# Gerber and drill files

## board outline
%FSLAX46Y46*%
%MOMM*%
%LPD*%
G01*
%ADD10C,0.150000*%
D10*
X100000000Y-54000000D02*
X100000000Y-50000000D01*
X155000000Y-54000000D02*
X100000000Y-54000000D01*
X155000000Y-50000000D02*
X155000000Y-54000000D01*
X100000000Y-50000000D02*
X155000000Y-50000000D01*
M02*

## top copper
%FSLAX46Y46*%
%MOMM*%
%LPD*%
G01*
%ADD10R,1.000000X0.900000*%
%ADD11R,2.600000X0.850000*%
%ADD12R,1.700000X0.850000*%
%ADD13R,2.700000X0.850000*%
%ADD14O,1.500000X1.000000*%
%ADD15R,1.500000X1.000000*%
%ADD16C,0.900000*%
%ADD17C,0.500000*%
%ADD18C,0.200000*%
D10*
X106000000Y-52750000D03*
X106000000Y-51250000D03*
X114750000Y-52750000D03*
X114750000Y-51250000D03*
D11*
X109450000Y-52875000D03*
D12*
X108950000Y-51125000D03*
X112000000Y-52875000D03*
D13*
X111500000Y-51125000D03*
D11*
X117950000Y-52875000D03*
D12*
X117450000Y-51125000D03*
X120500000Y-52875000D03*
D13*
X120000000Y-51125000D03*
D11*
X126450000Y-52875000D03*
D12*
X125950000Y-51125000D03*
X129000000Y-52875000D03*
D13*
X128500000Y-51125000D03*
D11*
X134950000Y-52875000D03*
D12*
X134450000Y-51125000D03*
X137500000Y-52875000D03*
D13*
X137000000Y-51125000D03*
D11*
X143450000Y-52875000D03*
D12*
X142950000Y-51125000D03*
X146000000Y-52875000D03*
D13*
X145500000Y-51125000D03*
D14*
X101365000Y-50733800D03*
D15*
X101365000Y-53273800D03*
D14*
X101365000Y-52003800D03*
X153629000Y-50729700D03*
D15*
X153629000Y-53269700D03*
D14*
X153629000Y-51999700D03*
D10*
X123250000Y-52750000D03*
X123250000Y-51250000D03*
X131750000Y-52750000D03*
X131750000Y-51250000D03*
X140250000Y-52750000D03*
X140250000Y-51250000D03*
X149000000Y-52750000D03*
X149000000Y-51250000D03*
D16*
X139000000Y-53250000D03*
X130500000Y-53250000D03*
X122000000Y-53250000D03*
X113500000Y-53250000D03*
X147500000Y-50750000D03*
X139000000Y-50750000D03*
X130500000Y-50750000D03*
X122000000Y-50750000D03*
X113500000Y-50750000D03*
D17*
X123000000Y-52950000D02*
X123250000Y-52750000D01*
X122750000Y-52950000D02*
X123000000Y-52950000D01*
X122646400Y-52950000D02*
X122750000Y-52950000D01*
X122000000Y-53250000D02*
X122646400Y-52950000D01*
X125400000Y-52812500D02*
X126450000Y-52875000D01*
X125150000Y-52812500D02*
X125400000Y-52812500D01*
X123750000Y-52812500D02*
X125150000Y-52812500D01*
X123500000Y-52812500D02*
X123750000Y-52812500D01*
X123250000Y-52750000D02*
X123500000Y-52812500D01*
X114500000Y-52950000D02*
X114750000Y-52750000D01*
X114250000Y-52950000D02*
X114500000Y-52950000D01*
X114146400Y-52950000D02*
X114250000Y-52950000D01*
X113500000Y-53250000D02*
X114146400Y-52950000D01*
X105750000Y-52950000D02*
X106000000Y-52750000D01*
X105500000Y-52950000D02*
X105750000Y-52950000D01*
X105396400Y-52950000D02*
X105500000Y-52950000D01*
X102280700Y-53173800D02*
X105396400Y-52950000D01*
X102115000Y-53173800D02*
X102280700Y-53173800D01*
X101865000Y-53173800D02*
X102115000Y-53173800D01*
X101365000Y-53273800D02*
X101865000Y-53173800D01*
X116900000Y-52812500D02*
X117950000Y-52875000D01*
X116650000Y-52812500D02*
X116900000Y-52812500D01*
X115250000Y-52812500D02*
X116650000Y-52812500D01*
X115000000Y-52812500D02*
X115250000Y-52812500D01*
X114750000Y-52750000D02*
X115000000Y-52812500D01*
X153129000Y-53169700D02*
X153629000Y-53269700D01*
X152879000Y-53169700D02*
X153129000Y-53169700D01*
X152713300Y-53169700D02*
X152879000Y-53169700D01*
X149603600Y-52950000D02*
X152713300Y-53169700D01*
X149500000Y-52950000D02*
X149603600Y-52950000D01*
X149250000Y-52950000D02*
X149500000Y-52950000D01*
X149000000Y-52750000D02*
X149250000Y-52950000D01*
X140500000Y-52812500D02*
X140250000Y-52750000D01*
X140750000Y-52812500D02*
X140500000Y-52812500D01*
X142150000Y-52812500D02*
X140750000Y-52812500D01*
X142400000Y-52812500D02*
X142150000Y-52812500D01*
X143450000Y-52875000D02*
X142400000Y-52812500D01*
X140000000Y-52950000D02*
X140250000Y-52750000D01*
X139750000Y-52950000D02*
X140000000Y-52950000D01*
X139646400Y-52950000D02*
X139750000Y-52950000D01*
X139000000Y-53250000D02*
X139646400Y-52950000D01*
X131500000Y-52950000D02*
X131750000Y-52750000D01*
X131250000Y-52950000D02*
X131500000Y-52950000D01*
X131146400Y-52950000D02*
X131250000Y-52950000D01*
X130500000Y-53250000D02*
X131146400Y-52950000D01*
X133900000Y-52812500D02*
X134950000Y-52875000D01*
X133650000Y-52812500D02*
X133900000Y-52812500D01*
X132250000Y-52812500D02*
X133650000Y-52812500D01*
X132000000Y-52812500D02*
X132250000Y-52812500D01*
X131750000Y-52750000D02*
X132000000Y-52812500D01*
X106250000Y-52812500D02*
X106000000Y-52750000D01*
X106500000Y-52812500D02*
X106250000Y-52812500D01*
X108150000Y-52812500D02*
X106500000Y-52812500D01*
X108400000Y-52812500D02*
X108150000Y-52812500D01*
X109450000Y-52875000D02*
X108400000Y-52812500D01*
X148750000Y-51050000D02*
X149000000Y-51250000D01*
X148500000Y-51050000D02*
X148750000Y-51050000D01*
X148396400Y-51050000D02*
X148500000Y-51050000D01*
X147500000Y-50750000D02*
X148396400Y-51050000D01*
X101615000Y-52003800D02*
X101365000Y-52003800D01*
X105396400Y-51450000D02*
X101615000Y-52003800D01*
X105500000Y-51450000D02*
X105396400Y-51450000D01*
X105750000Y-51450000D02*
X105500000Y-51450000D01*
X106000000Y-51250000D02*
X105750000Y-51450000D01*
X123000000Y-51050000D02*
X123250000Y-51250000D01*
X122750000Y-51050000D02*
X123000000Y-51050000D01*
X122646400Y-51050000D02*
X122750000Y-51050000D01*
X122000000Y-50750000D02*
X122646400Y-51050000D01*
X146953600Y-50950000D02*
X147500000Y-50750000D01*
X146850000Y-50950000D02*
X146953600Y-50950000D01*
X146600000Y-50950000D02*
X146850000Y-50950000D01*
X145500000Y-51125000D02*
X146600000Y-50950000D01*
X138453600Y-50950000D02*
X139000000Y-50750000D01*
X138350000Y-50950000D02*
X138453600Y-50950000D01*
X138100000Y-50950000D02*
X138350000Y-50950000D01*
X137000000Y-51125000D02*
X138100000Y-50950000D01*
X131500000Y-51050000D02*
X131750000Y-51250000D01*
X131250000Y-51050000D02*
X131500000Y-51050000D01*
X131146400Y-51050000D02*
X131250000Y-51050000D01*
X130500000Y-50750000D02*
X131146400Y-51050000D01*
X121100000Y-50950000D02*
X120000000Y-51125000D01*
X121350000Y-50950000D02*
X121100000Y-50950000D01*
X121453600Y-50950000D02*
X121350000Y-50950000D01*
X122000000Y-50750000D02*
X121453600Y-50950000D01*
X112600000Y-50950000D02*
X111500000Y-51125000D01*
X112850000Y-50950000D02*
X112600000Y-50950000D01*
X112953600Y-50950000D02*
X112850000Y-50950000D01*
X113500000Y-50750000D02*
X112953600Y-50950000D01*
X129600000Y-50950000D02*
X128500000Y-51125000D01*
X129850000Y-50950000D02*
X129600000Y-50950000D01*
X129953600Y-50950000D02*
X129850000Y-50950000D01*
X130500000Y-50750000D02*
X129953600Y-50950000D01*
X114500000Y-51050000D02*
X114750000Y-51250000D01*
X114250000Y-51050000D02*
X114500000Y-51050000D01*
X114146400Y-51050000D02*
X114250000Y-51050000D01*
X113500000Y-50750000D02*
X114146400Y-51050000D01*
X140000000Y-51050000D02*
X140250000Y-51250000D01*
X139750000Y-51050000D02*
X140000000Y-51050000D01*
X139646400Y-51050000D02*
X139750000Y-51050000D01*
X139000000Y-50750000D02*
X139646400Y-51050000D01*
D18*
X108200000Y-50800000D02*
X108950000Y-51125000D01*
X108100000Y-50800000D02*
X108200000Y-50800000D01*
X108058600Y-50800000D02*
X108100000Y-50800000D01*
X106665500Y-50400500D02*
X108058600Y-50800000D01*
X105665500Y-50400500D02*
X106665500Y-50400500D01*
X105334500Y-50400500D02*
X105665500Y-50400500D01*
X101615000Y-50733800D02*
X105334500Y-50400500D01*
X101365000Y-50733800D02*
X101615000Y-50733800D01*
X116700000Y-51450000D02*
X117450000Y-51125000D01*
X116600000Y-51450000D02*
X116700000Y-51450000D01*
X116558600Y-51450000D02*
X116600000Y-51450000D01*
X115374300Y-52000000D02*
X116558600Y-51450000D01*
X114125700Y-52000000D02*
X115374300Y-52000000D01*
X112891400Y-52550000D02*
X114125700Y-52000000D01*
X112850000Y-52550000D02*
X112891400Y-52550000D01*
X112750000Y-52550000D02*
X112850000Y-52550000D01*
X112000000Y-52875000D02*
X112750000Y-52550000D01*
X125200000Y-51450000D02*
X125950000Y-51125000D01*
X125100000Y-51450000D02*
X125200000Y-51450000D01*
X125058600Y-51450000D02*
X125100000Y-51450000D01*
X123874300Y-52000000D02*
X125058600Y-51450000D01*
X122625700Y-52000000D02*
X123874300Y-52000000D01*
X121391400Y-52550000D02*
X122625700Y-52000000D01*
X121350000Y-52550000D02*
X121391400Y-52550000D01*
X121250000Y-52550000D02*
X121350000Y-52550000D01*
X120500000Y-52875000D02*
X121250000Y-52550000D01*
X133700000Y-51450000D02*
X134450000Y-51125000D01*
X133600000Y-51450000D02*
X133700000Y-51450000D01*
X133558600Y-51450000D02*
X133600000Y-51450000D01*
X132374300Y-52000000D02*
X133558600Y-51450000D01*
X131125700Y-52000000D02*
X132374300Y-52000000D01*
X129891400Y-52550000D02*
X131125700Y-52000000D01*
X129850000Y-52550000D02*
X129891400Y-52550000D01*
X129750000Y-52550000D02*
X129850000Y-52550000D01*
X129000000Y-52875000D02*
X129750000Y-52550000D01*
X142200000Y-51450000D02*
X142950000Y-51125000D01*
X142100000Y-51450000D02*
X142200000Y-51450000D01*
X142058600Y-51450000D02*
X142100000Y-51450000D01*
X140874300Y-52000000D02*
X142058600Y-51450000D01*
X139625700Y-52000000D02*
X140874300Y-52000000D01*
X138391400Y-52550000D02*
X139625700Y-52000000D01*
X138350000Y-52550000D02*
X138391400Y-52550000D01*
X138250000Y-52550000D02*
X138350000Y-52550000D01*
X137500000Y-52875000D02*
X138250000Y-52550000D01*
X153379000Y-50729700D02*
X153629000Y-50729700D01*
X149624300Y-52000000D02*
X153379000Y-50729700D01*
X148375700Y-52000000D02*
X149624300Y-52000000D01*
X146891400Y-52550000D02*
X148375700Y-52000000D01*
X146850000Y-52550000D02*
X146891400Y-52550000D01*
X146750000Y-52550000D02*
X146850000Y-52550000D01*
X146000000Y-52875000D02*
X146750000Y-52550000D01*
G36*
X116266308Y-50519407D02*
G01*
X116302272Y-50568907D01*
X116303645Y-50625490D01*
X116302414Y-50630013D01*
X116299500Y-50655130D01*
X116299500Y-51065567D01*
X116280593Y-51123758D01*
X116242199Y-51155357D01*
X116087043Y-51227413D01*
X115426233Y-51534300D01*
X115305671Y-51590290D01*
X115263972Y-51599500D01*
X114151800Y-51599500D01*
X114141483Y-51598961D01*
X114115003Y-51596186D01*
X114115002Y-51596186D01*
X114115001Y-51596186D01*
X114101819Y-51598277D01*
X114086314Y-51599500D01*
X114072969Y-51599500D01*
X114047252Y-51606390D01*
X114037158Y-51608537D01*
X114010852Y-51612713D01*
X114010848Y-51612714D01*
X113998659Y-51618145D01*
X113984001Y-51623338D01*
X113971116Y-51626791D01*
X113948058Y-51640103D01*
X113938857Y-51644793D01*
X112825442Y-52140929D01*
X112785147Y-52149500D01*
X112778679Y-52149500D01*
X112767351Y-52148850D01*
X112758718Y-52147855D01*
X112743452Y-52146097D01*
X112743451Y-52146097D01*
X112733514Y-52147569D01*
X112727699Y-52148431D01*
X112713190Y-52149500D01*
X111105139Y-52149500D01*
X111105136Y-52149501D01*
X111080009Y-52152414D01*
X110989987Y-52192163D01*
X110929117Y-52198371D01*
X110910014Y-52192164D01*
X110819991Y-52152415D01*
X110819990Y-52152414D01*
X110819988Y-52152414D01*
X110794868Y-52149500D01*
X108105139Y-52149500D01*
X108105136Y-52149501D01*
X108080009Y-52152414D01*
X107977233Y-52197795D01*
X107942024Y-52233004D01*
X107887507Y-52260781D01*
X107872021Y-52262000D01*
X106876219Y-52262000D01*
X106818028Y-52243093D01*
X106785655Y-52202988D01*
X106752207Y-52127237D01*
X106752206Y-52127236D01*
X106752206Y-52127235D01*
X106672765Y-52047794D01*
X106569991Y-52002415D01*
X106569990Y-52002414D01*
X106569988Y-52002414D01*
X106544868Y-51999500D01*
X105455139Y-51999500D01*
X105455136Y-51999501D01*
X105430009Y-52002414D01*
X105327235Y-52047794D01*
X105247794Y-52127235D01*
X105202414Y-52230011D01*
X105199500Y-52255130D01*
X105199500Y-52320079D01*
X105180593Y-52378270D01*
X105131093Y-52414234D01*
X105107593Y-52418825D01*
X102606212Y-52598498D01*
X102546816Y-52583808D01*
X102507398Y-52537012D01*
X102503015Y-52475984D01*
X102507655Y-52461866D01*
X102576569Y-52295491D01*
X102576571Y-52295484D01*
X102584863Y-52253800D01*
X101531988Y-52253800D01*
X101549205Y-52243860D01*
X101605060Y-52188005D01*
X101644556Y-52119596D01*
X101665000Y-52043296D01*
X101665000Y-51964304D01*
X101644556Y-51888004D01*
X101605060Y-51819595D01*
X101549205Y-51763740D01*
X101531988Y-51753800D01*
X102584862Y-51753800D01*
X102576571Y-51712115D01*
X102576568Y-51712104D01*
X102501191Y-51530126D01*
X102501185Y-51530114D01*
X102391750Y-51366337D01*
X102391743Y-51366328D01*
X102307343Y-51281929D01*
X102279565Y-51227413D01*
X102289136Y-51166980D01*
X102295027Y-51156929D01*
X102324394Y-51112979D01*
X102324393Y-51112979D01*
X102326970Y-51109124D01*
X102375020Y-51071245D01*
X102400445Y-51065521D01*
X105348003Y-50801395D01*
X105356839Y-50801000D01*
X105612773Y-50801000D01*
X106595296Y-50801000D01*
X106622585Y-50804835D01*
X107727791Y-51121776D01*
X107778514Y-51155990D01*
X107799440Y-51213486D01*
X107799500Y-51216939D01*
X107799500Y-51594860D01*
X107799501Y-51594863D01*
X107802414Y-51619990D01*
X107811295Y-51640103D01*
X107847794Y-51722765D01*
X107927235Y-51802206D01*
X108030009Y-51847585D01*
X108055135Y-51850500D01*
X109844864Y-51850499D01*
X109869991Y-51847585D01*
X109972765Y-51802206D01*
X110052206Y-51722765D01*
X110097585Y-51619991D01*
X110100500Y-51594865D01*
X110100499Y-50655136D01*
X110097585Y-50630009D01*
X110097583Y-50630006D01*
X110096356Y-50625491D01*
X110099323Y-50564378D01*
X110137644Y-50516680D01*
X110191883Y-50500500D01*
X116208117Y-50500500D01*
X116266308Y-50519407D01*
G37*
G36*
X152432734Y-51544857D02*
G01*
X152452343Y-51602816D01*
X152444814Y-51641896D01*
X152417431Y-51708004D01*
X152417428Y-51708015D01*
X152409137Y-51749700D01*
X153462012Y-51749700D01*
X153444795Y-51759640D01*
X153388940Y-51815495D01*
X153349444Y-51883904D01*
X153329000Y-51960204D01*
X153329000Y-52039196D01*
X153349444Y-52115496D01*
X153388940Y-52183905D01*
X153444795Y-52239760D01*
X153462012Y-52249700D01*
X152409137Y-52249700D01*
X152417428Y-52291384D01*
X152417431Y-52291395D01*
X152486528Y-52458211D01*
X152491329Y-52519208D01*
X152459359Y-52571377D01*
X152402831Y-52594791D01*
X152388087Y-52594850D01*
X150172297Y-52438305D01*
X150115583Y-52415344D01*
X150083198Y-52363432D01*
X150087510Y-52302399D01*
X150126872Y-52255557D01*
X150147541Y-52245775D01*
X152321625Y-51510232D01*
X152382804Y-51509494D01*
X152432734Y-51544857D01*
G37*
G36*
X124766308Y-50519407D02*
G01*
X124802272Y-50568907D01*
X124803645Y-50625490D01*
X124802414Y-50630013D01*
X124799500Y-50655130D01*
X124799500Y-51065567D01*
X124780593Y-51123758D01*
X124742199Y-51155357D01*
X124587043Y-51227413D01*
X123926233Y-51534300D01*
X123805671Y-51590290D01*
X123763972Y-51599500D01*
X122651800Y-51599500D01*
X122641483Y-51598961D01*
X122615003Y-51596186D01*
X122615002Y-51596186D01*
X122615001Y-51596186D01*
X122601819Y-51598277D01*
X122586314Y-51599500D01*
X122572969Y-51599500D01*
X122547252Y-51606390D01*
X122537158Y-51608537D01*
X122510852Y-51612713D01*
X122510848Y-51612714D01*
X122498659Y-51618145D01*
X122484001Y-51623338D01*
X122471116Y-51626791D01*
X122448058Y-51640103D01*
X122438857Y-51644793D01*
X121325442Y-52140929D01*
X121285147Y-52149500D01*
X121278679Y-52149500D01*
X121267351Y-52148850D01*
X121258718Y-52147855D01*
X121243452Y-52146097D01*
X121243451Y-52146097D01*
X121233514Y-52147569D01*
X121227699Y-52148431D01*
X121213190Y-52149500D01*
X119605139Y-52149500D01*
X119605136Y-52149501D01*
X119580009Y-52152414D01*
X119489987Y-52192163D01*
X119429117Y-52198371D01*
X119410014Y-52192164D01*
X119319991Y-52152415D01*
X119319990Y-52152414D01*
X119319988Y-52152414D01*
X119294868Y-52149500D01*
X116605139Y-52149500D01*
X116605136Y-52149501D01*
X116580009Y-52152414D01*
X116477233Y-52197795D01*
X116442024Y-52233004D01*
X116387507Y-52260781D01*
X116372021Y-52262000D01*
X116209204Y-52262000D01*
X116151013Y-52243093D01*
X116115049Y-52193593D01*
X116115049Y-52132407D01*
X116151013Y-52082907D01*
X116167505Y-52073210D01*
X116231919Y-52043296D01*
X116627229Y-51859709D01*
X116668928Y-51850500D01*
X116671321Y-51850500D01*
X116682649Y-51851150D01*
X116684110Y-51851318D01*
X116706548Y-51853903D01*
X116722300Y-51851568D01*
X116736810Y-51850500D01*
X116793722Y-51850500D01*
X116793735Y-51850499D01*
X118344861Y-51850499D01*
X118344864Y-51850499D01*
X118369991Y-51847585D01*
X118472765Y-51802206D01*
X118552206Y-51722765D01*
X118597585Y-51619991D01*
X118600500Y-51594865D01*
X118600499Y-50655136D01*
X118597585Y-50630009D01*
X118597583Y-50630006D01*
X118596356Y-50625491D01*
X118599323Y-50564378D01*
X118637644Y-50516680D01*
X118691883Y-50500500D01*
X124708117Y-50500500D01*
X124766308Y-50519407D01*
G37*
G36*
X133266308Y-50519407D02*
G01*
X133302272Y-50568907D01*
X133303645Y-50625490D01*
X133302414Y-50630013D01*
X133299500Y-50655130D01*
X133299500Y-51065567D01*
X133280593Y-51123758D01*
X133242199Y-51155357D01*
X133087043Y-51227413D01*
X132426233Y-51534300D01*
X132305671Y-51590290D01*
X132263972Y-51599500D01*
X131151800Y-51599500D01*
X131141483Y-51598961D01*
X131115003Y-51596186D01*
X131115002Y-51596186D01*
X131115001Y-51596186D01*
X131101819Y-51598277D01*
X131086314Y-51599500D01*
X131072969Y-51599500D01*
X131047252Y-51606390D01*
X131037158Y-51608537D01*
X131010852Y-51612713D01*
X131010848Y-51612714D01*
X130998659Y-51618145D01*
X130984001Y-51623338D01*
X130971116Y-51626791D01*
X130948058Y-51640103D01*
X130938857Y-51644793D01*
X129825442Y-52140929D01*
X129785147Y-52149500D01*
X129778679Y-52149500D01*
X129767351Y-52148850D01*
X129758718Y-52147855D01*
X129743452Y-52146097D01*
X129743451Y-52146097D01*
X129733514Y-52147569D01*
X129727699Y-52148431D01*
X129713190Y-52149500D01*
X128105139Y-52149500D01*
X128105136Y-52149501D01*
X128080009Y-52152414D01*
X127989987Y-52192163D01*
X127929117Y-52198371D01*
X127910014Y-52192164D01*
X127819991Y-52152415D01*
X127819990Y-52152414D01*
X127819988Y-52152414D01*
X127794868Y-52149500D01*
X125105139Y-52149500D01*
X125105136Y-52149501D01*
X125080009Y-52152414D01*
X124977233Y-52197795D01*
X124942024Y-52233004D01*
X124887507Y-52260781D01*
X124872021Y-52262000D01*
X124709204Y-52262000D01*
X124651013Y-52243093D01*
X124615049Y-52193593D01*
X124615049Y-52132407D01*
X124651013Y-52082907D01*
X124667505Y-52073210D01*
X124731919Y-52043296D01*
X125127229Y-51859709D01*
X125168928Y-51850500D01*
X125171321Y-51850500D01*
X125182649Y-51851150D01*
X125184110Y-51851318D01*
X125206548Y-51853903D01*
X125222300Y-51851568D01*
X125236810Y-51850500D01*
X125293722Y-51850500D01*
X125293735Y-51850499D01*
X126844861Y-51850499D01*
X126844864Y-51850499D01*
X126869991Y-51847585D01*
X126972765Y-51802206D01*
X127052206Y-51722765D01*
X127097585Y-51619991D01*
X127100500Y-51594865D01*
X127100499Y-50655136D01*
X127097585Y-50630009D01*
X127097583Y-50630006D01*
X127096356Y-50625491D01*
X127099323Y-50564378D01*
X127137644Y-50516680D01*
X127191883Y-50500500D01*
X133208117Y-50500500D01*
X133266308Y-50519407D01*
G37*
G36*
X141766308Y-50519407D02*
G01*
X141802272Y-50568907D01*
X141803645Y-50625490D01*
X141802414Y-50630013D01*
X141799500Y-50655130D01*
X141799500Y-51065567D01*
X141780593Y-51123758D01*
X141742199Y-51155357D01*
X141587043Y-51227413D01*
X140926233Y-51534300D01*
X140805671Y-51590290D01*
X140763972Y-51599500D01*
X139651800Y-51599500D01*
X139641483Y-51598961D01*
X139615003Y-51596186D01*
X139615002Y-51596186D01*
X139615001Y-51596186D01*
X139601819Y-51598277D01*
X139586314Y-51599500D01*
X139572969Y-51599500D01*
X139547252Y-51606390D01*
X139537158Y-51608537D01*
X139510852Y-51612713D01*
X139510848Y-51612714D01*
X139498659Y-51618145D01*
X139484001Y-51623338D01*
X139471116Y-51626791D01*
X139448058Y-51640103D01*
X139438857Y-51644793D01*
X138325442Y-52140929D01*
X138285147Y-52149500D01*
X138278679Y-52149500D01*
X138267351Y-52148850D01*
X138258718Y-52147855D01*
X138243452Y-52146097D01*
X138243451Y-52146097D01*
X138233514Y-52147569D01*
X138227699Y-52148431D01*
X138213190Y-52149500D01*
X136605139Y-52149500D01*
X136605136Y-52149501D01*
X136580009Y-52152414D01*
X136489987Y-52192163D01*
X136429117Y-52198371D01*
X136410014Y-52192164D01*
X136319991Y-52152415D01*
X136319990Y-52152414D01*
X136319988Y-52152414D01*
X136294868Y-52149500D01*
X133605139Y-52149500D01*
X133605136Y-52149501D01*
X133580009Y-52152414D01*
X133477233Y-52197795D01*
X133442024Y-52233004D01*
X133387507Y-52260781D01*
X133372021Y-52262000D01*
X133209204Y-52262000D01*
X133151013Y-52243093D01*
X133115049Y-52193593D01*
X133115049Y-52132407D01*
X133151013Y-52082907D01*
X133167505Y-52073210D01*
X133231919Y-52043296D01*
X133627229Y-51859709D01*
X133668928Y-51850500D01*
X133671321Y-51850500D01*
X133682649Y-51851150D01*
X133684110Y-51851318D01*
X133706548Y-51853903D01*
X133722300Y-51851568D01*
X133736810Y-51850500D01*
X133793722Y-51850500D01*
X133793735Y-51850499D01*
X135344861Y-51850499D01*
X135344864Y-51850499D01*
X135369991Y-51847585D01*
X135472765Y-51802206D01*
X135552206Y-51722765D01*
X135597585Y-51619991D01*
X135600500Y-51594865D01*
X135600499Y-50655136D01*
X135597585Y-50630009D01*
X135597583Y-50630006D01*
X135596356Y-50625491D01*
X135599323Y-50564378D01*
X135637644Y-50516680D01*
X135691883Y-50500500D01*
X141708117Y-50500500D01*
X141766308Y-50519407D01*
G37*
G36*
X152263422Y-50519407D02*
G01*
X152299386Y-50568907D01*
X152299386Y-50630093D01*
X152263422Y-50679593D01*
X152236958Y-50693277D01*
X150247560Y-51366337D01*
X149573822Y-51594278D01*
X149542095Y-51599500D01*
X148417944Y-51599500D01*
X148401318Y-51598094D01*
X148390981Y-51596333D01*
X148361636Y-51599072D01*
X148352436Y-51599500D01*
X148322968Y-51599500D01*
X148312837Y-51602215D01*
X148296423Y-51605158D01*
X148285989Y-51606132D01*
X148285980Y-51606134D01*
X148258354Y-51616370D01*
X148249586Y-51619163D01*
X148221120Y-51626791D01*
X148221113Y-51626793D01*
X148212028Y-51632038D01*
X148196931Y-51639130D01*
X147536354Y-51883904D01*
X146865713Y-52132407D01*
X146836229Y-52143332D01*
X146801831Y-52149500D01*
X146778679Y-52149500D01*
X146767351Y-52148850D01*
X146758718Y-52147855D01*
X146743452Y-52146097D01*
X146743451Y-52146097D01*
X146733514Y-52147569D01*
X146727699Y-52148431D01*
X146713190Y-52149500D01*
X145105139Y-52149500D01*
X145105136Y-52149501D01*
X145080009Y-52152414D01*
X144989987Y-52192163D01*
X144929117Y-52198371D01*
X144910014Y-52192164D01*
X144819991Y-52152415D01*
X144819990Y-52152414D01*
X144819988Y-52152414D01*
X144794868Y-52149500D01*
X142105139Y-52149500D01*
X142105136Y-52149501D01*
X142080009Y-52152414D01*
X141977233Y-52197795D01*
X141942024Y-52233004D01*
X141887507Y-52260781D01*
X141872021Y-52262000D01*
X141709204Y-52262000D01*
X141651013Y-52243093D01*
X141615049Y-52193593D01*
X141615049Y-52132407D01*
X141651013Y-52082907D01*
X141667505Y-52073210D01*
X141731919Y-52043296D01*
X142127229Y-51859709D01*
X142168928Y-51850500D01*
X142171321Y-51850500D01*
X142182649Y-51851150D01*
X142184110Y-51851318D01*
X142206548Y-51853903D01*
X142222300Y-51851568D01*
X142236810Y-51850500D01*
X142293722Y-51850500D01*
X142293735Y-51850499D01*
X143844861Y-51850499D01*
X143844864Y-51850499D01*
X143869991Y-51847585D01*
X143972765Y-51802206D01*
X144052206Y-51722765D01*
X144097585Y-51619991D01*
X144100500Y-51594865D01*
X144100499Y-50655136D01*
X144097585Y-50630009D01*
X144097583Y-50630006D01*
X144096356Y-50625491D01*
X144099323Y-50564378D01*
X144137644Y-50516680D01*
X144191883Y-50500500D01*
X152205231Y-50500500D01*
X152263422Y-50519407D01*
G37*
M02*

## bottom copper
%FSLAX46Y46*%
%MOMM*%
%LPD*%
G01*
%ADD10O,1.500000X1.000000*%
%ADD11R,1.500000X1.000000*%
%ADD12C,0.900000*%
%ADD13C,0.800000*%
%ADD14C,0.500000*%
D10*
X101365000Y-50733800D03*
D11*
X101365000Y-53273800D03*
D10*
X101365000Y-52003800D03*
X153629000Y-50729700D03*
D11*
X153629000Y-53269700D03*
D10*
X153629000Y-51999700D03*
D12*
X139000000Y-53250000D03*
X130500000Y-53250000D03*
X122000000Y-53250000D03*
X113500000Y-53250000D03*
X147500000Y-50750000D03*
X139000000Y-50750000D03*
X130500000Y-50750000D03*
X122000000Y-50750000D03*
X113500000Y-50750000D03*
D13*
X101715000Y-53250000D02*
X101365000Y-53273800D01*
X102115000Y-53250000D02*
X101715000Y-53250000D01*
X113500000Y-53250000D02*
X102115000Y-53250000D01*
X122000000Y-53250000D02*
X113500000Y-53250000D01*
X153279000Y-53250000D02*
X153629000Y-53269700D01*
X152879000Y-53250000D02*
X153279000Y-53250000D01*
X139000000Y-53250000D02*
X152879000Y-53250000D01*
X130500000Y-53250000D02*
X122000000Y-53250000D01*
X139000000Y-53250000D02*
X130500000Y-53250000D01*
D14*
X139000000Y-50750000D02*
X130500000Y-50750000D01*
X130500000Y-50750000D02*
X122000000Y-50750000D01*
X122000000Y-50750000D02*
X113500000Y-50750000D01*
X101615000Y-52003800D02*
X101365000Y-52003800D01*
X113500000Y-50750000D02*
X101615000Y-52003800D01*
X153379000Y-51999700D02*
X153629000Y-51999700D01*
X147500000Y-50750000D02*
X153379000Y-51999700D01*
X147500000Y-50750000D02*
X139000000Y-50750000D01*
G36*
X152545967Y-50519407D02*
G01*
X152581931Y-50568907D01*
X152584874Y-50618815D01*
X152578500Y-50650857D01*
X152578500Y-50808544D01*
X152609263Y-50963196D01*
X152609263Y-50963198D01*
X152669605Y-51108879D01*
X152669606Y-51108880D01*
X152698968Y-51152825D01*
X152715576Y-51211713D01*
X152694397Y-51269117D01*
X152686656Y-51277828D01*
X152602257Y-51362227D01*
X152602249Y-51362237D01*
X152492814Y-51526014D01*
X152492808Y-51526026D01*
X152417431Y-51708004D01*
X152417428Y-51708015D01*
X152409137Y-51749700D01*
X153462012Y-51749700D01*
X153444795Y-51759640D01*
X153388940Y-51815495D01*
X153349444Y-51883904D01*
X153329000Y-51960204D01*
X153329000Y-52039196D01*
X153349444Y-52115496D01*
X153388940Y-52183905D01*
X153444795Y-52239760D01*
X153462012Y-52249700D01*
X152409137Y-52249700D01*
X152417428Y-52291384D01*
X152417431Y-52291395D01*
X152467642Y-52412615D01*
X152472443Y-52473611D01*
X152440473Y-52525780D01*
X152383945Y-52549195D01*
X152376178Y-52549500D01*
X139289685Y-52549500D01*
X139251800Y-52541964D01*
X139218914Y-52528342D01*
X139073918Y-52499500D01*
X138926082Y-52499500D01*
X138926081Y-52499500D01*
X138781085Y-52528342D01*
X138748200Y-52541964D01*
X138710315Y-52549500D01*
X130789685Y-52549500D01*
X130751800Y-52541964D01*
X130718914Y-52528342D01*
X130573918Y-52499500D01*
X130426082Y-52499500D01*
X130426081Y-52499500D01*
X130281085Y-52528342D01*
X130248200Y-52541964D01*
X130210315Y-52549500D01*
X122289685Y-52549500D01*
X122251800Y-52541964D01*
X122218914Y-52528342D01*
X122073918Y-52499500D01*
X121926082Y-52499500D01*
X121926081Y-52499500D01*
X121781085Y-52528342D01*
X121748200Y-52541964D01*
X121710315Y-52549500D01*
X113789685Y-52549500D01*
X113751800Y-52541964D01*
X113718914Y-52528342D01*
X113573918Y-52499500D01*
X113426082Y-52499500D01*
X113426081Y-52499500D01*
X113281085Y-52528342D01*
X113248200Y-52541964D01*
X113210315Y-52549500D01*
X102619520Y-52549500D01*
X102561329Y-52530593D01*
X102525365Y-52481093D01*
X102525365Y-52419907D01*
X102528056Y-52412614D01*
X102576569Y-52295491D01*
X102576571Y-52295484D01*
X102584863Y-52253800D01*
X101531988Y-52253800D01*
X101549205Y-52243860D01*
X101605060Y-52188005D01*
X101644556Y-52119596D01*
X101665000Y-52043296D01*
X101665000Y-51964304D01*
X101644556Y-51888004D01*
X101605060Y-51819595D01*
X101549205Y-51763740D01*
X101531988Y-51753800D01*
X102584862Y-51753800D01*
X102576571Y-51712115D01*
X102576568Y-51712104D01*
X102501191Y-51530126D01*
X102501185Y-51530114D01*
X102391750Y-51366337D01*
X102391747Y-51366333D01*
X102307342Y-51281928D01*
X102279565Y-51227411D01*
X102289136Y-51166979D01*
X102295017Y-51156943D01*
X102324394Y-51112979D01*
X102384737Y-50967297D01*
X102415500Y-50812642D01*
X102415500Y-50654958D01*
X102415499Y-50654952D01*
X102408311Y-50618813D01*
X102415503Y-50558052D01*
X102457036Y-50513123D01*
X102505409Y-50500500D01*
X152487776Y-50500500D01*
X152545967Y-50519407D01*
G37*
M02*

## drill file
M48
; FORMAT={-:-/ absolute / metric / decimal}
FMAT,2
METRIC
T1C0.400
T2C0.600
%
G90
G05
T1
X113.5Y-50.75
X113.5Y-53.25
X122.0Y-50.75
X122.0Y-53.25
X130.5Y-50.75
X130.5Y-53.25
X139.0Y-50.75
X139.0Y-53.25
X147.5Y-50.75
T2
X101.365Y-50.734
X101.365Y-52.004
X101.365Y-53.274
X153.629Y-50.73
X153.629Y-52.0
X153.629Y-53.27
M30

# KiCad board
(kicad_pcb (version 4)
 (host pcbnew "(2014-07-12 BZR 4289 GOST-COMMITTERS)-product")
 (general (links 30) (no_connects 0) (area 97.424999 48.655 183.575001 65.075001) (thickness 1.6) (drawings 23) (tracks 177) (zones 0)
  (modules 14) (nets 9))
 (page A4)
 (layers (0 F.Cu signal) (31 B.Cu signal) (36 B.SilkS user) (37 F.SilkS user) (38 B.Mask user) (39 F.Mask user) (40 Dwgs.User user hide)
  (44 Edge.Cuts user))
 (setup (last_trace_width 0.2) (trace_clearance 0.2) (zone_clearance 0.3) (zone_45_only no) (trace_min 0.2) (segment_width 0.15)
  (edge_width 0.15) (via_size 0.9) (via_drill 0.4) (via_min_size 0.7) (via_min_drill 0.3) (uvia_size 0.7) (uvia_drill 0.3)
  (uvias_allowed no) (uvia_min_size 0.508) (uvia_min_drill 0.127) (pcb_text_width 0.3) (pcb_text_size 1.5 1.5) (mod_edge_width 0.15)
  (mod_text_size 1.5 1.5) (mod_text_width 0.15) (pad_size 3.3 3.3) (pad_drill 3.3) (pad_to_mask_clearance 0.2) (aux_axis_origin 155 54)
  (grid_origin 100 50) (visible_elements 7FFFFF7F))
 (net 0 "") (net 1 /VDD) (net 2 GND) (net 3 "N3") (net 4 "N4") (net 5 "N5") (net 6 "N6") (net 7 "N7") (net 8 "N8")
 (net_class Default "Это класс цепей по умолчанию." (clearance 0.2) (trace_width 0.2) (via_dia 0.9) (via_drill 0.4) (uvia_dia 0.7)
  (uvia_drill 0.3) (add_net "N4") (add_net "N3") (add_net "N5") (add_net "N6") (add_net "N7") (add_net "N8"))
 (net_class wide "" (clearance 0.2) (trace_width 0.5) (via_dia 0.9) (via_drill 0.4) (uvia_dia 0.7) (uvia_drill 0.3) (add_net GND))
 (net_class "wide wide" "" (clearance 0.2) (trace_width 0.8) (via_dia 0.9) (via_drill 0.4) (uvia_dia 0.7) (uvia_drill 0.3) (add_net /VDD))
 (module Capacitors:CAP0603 (layer F.Cu) (at 106 52 90)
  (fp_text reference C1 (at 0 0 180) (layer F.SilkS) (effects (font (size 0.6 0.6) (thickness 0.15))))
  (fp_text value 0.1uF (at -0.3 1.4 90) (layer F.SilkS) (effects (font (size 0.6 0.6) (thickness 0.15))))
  (pad 1 smd rect (at -0.75 0 90) (size 0.9 1) (layers F.Cu F.Mask) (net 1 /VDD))
  (pad 2 smd rect (at 0.75 0 90) (size 0.9 1) (layers F.Cu F.Mask) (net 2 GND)))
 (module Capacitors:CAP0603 (layer F.Cu) (at 114.75 52 90)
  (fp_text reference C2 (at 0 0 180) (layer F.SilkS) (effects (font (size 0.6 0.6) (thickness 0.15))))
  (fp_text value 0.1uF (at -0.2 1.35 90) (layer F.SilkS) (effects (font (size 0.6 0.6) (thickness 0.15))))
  (pad 1 smd rect (at -0.75 0 90) (size 0.9 1) (layers F.Cu F.Mask) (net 1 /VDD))
  (pad 2 smd rect (at 0.75 0 90) (size 0.9 1) (layers F.Cu F.Mask) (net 2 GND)))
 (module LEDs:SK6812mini (layer F.Cu) (at 110.5 52 180)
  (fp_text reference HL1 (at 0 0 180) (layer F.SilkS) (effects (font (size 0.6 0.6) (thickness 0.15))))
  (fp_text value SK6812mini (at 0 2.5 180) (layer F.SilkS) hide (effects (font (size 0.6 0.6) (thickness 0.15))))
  (pad 4 smd rect (at 1.05 -0.875 180) (size 2.6 0.85) (layers F.Cu F.Mask) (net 1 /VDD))
  (pad 3 smd rect (at 1.55 0.875 180) (size 1.7 0.85) (layers F.Cu F.Mask) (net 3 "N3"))
  (pad 1 smd rect (at -1.5 -0.875 180) (size 1.7 0.85) (layers F.Cu F.Mask) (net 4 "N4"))
  (pad 2 smd rect (at -1 0.875 180) (size 2.7 0.85) (layers F.Cu F.Mask) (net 2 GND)))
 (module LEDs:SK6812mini (layer F.Cu) (at 119 52 180)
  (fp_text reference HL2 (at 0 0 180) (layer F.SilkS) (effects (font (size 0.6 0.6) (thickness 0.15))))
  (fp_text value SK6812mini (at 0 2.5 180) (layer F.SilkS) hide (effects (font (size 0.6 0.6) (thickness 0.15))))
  (pad 4 smd rect (at 1.05 -0.875 180) (size 2.6 0.85) (layers F.Cu F.Mask) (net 1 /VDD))
  (pad 3 smd rect (at 1.55 0.875 180) (size 1.7 0.85) (layers F.Cu F.Mask) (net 4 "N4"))
  (pad 1 smd rect (at -1.5 -0.875 180) (size 1.7 0.85) (layers F.Cu F.Mask) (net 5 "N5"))
  (pad 2 smd rect (at -1 0.875 180) (size 2.7 0.85) (layers F.Cu F.Mask) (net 2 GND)))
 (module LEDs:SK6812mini (layer F.Cu) (at 127.5 52 180)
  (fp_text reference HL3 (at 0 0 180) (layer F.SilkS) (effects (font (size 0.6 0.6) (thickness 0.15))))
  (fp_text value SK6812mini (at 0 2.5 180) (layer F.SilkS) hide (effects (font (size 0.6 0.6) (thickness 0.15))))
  (pad 4 smd rect (at 1.05 -0.875 180) (size 2.6 0.85) (layers F.Cu F.Mask) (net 1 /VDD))
  (pad 3 smd rect (at 1.55 0.875 180) (size 1.7 0.85) (layers F.Cu F.Mask) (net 5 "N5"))
  (pad 1 smd rect (at -1.5 -0.875 180) (size 1.7 0.85) (layers F.Cu F.Mask) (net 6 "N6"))
  (pad 2 smd rect (at -1 0.875 180) (size 2.7 0.85) (layers F.Cu F.Mask) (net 2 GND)))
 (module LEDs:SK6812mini (layer F.Cu) (at 136 52 180)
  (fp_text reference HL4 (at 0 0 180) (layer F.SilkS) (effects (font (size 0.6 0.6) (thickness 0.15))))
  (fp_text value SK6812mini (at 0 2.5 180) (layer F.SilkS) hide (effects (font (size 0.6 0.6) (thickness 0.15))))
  (pad 4 smd rect (at 1.05 -0.875 180) (size 2.6 0.85) (layers F.Cu F.Mask) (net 1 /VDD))
  (pad 3 smd rect (at 1.55 0.875 180) (size 1.7 0.85) (layers F.Cu F.Mask) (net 6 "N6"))
  (pad 1 smd rect (at -1.5 -0.875 180) (size 1.7 0.85) (layers F.Cu F.Mask) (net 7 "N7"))
  (pad 2 smd rect (at -1 0.875 180) (size 2.7 0.85) (layers F.Cu F.Mask) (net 2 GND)))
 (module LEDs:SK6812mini (layer F.Cu) (at 144.5 52 180)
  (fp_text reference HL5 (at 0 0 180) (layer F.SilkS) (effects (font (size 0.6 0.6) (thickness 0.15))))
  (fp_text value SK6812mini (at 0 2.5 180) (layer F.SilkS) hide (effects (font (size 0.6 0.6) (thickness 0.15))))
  (pad 4 smd rect (at 1.05 -0.875 180) (size 2.6 0.85) (layers F.Cu F.Mask) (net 1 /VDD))
  (pad 3 smd rect (at 1.55 0.875 180) (size 1.7 0.85) (layers F.Cu F.Mask) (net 7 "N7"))
  (pad 1 smd rect (at -1.5 -0.875 180) (size 1.7 0.85) (layers F.Cu F.Mask) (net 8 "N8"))
  (pad 2 smd rect (at -1 0.875 180) (size 2.7 0.85) (layers F.Cu F.Mask) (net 2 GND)))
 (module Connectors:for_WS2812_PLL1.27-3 (layer F.Cu) (at 101.365 53.2738 90)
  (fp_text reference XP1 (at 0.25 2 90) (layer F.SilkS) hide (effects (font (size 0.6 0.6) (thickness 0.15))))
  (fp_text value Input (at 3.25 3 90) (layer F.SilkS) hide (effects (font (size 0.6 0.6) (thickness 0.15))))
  (pad 3 thru_hole oval (at 2.54 0 90) (size 1 1.5) (drill 0.6) (layers *.Cu *.Mask) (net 3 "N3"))
  (pad 1 thru_hole rect (at 0 0 90) (size 1 1.5) (drill 0.6) (layers *.Cu *.Mask) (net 1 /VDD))
  (pad 2 thru_hole oval (at 1.27 0 90) (size 1 1.5) (drill 0.6) (layers *.Cu *.Mask) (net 2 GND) (zone_connect 1)))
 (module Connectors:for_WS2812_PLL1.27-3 (layer F.Cu) (at 153.629 53.2697 90)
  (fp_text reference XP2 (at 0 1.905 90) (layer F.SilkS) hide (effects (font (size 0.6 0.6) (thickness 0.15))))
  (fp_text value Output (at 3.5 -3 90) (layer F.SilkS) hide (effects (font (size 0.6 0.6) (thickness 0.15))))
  (pad 3 thru_hole oval (at 2.54 0 90) (size 1 1.5) (drill 0.6) (layers *.Cu *.Mask) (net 8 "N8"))
  (pad 1 thru_hole rect (at 0 0 90) (size 1 1.5) (drill 0.6) (layers *.Cu *.Mask) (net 1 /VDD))
  (pad 2 thru_hole oval (at 1.27 0 90) (size 1 1.5) (drill 0.6) (layers *.Cu *.Mask) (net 2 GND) (zone_connect 1)))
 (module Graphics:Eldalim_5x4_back (layer B.Cu) (at 117.5 52)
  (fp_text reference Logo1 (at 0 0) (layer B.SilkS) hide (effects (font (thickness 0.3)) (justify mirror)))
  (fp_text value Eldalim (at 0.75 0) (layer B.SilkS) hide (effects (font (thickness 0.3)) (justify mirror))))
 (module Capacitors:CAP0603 (layer F.Cu) (at 123.25 52 90)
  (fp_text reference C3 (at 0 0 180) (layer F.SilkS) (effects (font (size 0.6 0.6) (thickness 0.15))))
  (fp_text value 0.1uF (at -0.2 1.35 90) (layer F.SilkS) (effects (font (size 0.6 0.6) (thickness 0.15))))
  (pad 1 smd rect (at -0.75 0 90) (size 0.9 1) (layers F.Cu F.Mask) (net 1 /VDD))
  (pad 2 smd rect (at 0.75 0 90) (size 0.9 1) (layers F.Cu F.Mask) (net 2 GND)))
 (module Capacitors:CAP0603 (layer F.Cu) (at 131.75 52 90)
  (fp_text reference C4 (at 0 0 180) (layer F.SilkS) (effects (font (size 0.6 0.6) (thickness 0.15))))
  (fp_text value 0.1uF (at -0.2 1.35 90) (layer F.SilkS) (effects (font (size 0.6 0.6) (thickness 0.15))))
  (pad 1 smd rect (at -0.75 0 90) (size 0.9 1) (layers F.Cu F.Mask) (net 1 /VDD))
  (pad 2 smd rect (at 0.75 0 90) (size 0.9 1) (layers F.Cu F.Mask) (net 2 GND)))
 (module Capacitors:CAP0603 (layer F.Cu) (at 140.25 52 90)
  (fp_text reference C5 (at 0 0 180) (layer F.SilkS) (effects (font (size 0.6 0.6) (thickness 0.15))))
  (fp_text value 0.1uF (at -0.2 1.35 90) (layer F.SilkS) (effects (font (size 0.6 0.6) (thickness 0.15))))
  (pad 1 smd rect (at -0.75 0 90) (size 0.9 1) (layers F.Cu F.Mask) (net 1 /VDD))
  (pad 2 smd rect (at 0.75 0 90) (size 0.9 1) (layers F.Cu F.Mask) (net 2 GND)))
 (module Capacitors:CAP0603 (layer F.Cu) (at 149 52 90)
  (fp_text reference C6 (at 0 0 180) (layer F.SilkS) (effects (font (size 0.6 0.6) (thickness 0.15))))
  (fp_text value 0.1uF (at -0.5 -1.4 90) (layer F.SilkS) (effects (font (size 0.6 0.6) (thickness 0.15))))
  (pad 1 smd rect (at -0.75 0 90) (size 0.9 1) (layers F.Cu F.Mask) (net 1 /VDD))
  (pad 2 smd rect (at 0.75 0 90) (size 0.9 1) (layers F.Cu F.Mask) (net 2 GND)))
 (gr_line (start 100 54) (end 100 50) (angle 90) (layer Edge.Cuts) (width 0.15))
 (gr_line (start 155 54) (end 100 54) (angle 90) (layer Edge.Cuts) (width 0.15))
 (gr_line (start 155 50) (end 155 54) (angle 90) (layer Edge.Cuts) (width 0.15))
 (gr_line (start 100 50) (end 155 50) (angle 90) (layer Edge.Cuts) (width 0.15)) (via (at 139 53.25) (size 0.9) (layers F.Cu B.Cu) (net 1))
 (via (at 130.5 53.25) (size 0.9) (layers F.Cu B.Cu) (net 1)) (via (at 122 53.25) (size 0.9) (layers F.Cu B.Cu) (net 1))
 (via (at 113.5 53.25) (size 0.9) (layers F.Cu B.Cu) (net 1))
 (segment (start 101.715 53.25) (end 101.365 53.2738) (width 0.8) (layer B.Cu) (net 1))
 (segment (start 102.115 53.25) (end 101.715 53.25) (width 0.8) (layer B.Cu) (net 1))
 (segment (start 113.5 53.25) (end 102.115 53.25) (width 0.8) (layer B.Cu) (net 1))
 (segment (start 122 53.25) (end 113.5 53.25) (width 0.8) (layer B.Cu) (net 1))
 (segment (start 153.279 53.25) (end 153.629 53.2697) (width 0.8) (layer B.Cu) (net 1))
 (segment (start 152.879 53.25) (end 153.279 53.25) (width 0.8) (layer B.Cu) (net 1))
 (segment (start 139 53.25) (end 152.879 53.25) (width 0.8) (layer B.Cu) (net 1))
 (segment (start 130.5 53.25) (end 122 53.25) (width 0.8) (layer B.Cu) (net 1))
 (segment (start 139 53.25) (end 130.5 53.25) (width 0.8) (layer B.Cu) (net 1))
 (segment (start 123 52.95) (end 123.25 52.75) (width 0.5) (layer F.Cu) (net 1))
 (segment (start 122.75 52.95) (end 123 52.95) (width 0.5) (layer F.Cu) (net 1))
 (segment (start 122.6464 52.95) (end 122.75 52.95) (width 0.5) (layer F.Cu) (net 1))
 (segment (start 122 53.25) (end 122.6464 52.95) (width 0.5) (layer F.Cu) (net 1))
 (segment (start 125.4 52.8125) (end 126.45 52.875) (width 0.5) (layer F.Cu) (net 1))
 (segment (start 125.15 52.8125) (end 125.4 52.8125) (width 0.5) (layer F.Cu) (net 1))
 (segment (start 123.75 52.8125) (end 125.15 52.8125) (width 0.5) (layer F.Cu) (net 1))
 (segment (start 123.5 52.8125) (end 123.75 52.8125) (width 0.5) (layer F.Cu) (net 1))
 (segment (start 123.25 52.75) (end 123.5 52.8125) (width 0.5) (layer F.Cu) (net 1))
 (segment (start 114.5 52.95) (end 114.75 52.75) (width 0.5) (layer F.Cu) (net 1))
 (segment (start 114.25 52.95) (end 114.5 52.95) (width 0.5) (layer F.Cu) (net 1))
 (segment (start 114.1464 52.95) (end 114.25 52.95) (width 0.5) (layer F.Cu) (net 1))
 (segment (start 113.5 53.25) (end 114.1464 52.95) (width 0.5) (layer F.Cu) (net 1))
 (segment (start 105.75 52.95) (end 106 52.75) (width 0.5) (layer F.Cu) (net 1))
 (segment (start 105.5 52.95) (end 105.75 52.95) (width 0.5) (layer F.Cu) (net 1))
 (segment (start 105.3964 52.95) (end 105.5 52.95) (width 0.5) (layer F.Cu) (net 1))
 (segment (start 102.2807 53.1738) (end 105.3964 52.95) (width 0.5) (layer F.Cu) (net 1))
 (segment (start 102.115 53.1738) (end 102.2807 53.1738) (width 0.5) (layer F.Cu) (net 1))
 (segment (start 101.865 53.1738) (end 102.115 53.1738) (width 0.5) (layer F.Cu) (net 1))
 (segment (start 101.365 53.2738) (end 101.865 53.1738) (width 0.5) (layer F.Cu) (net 1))
 (segment (start 116.9 52.8125) (end 117.95 52.875) (width 0.5) (layer F.Cu) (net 1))
 (segment (start 116.65 52.8125) (end 116.9 52.8125) (width 0.5) (layer F.Cu) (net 1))
 (segment (start 115.25 52.8125) (end 116.65 52.8125) (width 0.5) (layer F.Cu) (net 1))
 (segment (start 115 52.8125) (end 115.25 52.8125) (width 0.5) (layer F.Cu) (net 1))
 (segment (start 114.75 52.75) (end 115 52.8125) (width 0.5) (layer F.Cu) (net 1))
 (segment (start 153.129 53.1697) (end 153.629 53.2697) (width 0.5) (layer F.Cu) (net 1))
 (segment (start 152.879 53.1697) (end 153.129 53.1697) (width 0.5) (layer F.Cu) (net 1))
 (segment (start 152.7133 53.1697) (end 152.879 53.1697) (width 0.5) (layer F.Cu) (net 1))
 (segment (start 149.6036 52.95) (end 152.7133 53.1697) (width 0.5) (layer F.Cu) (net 1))
 (segment (start 149.5 52.95) (end 149.6036 52.95) (width 0.5) (layer F.Cu) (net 1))
 (segment (start 149.25 52.95) (end 149.5 52.95) (width 0.5) (layer F.Cu) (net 1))
 (segment (start 149 52.75) (end 149.25 52.95) (width 0.5) (layer F.Cu) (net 1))
 (segment (start 140.5 52.8125) (end 140.25 52.75) (width 0.5) (layer F.Cu) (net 1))
 (segment (start 140.75 52.8125) (end 140.5 52.8125) (width 0.5) (layer F.Cu) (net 1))
 (segment (start 142.15 52.8125) (end 140.75 52.8125) (width 0.5) (layer F.Cu) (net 1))
 (segment (start 142.4 52.8125) (end 142.15 52.8125) (width 0.5) (layer F.Cu) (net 1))
 (segment (start 143.45 52.875) (end 142.4 52.8125) (width 0.5) (layer F.Cu) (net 1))
 (segment (start 140 52.95) (end 140.25 52.75) (width 0.5) (layer F.Cu) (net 1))
 (segment (start 139.75 52.95) (end 140 52.95) (width 0.5) (layer F.Cu) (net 1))
 (segment (start 139.6464 52.95) (end 139.75 52.95) (width 0.5) (layer F.Cu) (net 1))
 (segment (start 139 53.25) (end 139.6464 52.95) (width 0.5) (layer F.Cu) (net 1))
 (segment (start 131.5 52.95) (end 131.75 52.75) (width 0.5) (layer F.Cu) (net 1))
 (segment (start 131.25 52.95) (end 131.5 52.95) (width 0.5) (layer F.Cu) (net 1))
 (segment (start 131.1464 52.95) (end 131.25 52.95) (width 0.5) (layer F.Cu) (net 1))
 (segment (start 130.5 53.25) (end 131.1464 52.95) (width 0.5) (layer F.Cu) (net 1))
 (segment (start 133.9 52.8125) (end 134.95 52.875) (width 0.5) (layer F.Cu) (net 1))
 (segment (start 133.65 52.8125) (end 133.9 52.8125) (width 0.5) (layer F.Cu) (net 1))
 (segment (start 132.25 52.8125) (end 133.65 52.8125) (width 0.5) (layer F.Cu) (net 1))
 (segment (start 132 52.8125) (end 132.25 52.8125) (width 0.5) (layer F.Cu) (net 1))
 (segment (start 131.75 52.75) (end 132 52.8125) (width 0.5) (layer F.Cu) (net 1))
 (segment (start 106.25 52.8125) (end 106 52.75) (width 0.5) (layer F.Cu) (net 1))
 (segment (start 106.5 52.8125) (end 106.25 52.8125) (width 0.5) (layer F.Cu) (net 1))
 (segment (start 108.15 52.8125) (end 106.5 52.8125) (width 0.5) (layer F.Cu) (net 1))
 (segment (start 108.4 52.8125) (end 108.15 52.8125) (width 0.5) (layer F.Cu) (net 1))
 (segment (start 109.45 52.875) (end 108.4 52.8125) (width 0.5) (layer F.Cu) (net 1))
 (via (at 147.5 50.75) (size 0.9) (layers F.Cu B.Cu) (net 2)) (via (at 139 50.75) (size 0.9) (layers F.Cu B.Cu) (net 2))
 (via (at 130.5 50.75) (size 0.9) (layers F.Cu B.Cu) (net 2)) (via (at 122 50.75) (size 0.9) (layers F.Cu B.Cu) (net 2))
 (via (at 113.5 50.75) (size 0.9) (layers F.Cu B.Cu) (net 2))
 (segment (start 139 50.75) (end 130.5 50.75) (width 0.5) (layer B.Cu) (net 2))
 (segment (start 130.5 50.75) (end 122 50.75) (width 0.5) (layer B.Cu) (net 2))
 (segment (start 122 50.75) (end 113.5 50.75) (width 0.5) (layer B.Cu) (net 2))
 (segment (start 101.615 52.0038) (end 101.365 52.0038) (width 0.5) (layer B.Cu) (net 2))
 (segment (start 113.5 50.75) (end 101.615 52.0038) (width 0.5) (layer B.Cu) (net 2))
 (segment (start 153.379 51.9997) (end 153.629 51.9997) (width 0.5) (layer B.Cu) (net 2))
 (segment (start 147.5 50.75) (end 153.379 51.9997) (width 0.5) (layer B.Cu) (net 2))
 (segment (start 147.5 50.75) (end 139 50.75) (width 0.5) (layer B.Cu) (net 2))
 (segment (start 148.75 51.05) (end 149 51.25) (width 0.5) (layer F.Cu) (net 2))
 (segment (start 148.5 51.05) (end 148.75 51.05) (width 0.5) (layer F.Cu) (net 2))
 (segment (start 148.3964 51.05) (end 148.5 51.05) (width 0.5) (layer F.Cu) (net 2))
 (segment (start 147.5 50.75) (end 148.3964 51.05) (width 0.5) (layer F.Cu) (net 2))
 (segment (start 101.615 52.0038) (end 101.365 52.0038) (width 0.5) (layer F.Cu) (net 2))
 (segment (start 105.3964 51.45) (end 101.615 52.0038) (width 0.5) (layer F.Cu) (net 2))
 (segment (start 105.5 51.45) (end 105.3964 51.45) (width 0.5) (layer F.Cu) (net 2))
 (segment (start 105.75 51.45) (end 105.5 51.45) (width 0.5) (layer F.Cu) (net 2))
 (segment (start 106 51.25) (end 105.75 51.45) (width 0.5) (layer F.Cu) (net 2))
 (segment (start 123 51.05) (end 123.25 51.25) (width 0.5) (layer F.Cu) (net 2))
 (segment (start 122.75 51.05) (end 123 51.05) (width 0.5) (layer F.Cu) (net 2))
 (segment (start 122.6464 51.05) (end 122.75 51.05) (width 0.5) (layer F.Cu) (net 2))
 (segment (start 122 50.75) (end 122.6464 51.05) (width 0.5) (layer F.Cu) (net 2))
 (segment (start 146.9536 50.95) (end 147.5 50.75) (width 0.5) (layer F.Cu) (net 2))
 (segment (start 146.85 50.95) (end 146.9536 50.95) (width 0.5) (layer F.Cu) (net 2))
 (segment (start 146.6 50.95) (end 146.85 50.95) (width 0.5) (layer F.Cu) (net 2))
 (segment (start 145.5 51.125) (end 146.6 50.95) (width 0.5) (layer F.Cu) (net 2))
 (segment (start 138.4536 50.95) (end 139 50.75) (width 0.5) (layer F.Cu) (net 2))
 (segment (start 138.35 50.95) (end 138.4536 50.95) (width 0.5) (layer F.Cu) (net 2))
 (segment (start 138.1 50.95) (end 138.35 50.95) (width 0.5) (layer F.Cu) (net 2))
 (segment (start 137 51.125) (end 138.1 50.95) (width 0.5) (layer F.Cu) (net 2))
 (segment (start 131.5 51.05) (end 131.75 51.25) (width 0.5) (layer F.Cu) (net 2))
 (segment (start 131.25 51.05) (end 131.5 51.05) (width 0.5) (layer F.Cu) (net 2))
 (segment (start 131.1464 51.05) (end 131.25 51.05) (width 0.5) (layer F.Cu) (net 2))
 (segment (start 130.5 50.75) (end 131.1464 51.05) (width 0.5) (layer F.Cu) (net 2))
 (segment (start 121.1 50.95) (end 120 51.125) (width 0.5) (layer F.Cu) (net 2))
 (segment (start 121.35 50.95) (end 121.1 50.95) (width 0.5) (layer F.Cu) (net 2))
 (segment (start 121.4536 50.95) (end 121.35 50.95) (width 0.5) (layer F.Cu) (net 2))
 (segment (start 122 50.75) (end 121.4536 50.95) (width 0.5) (layer F.Cu) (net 2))
 (segment (start 112.6 50.95) (end 111.5 51.125) (width 0.5) (layer F.Cu) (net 2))
 (segment (start 112.85 50.95) (end 112.6 50.95) (width 0.5) (layer F.Cu) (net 2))
 (segment (start 112.9536 50.95) (end 112.85 50.95) (width 0.5) (layer F.Cu) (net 2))
 (segment (start 113.5 50.75) (end 112.9536 50.95) (width 0.5) (layer F.Cu) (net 2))
 (segment (start 129.6 50.95) (end 128.5 51.125) (width 0.5) (layer F.Cu) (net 2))
 (segment (start 129.85 50.95) (end 129.6 50.95) (width 0.5) (layer F.Cu) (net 2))
 (segment (start 129.9536 50.95) (end 129.85 50.95) (width 0.5) (layer F.Cu) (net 2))
 (segment (start 130.5 50.75) (end 129.9536 50.95) (width 0.5) (layer F.Cu) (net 2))
 (segment (start 114.5 51.05) (end 114.75 51.25) (width 0.5) (layer F.Cu) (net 2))
 (segment (start 114.25 51.05) (end 114.5 51.05) (width 0.5) (layer F.Cu) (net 2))
 (segment (start 114.1464 51.05) (end 114.25 51.05) (width 0.5) (layer F.Cu) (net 2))
 (segment (start 113.5 50.75) (end 114.1464 51.05) (width 0.5) (layer F.Cu) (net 2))
 (segment (start 140 51.05) (end 140.25 51.25) (width 0.5) (layer F.Cu) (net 2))
 (segment (start 139.75 51.05) (end 140 51.05) (width 0.5) (layer F.Cu) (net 2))
 (segment (start 139.6464 51.05) (end 139.75 51.05) (width 0.5) (layer F.Cu) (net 2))
 (segment (start 139 50.75) (end 139.6464 51.05) (width 0.5) (layer F.Cu) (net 2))
 (segment (start 108.2 50.8) (end 108.95 51.125) (width 0.2) (layer F.Cu) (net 3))
 (segment (start 108.1 50.8) (end 108.2 50.8) (width 0.2) (layer F.Cu) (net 3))
 (segment (start 108.0586 50.8) (end 108.1 50.8) (width 0.2) (layer F.Cu) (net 3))
 (segment (start 106.6655 50.4005) (end 108.0586 50.8) (width 0.2) (layer F.Cu) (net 3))
 (segment (start 105.6655 50.4005) (end 106.6655 50.4005) (width 0.2) (layer F.Cu) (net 3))
 (segment (start 105.3345 50.4005) (end 105.6655 50.4005) (width 0.2) (layer F.Cu) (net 3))
 (segment (start 101.615 50.7338) (end 105.3345 50.4005) (width 0.2) (layer F.Cu) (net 3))
 (segment (start 101.365 50.7338) (end 101.615 50.7338) (width 0.2) (layer F.Cu) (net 3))
 (segment (start 116.7 51.45) (end 117.45 51.125) (width 0.2) (layer F.Cu) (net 4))
 (segment (start 116.6 51.45) (end 116.7 51.45) (width 0.2) (layer F.Cu) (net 4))
 (segment (start 116.5586 51.45) (end 116.6 51.45) (width 0.2) (layer F.Cu) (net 4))
 (segment (start 115.3743 52) (end 116.5586 51.45) (width 0.2) (layer F.Cu) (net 4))
 (segment (start 114.1257 52) (end 115.3743 52) (width 0.2) (layer F.Cu) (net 4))
 (segment (start 112.8914 52.55) (end 114.1257 52) (width 0.2) (layer F.Cu) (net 4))
 (segment (start 112.85 52.55) (end 112.8914 52.55) (width 0.2) (layer F.Cu) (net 4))
 (segment (start 112.75 52.55) (end 112.85 52.55) (width 0.2) (layer F.Cu) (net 4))
 (segment (start 112 52.875) (end 112.75 52.55) (width 0.2) (layer F.Cu) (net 4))
 (segment (start 125.2 51.45) (end 125.95 51.125) (width 0.2) (layer F.Cu) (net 5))
 (segment (start 125.1 51.45) (end 125.2 51.45) (width 0.2) (layer F.Cu) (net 5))
 (segment (start 125.0586 51.45) (end 125.1 51.45) (width 0.2) (layer F.Cu) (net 5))
 (segment (start 123.8743 52) (end 125.0586 51.45) (width 0.2) (layer F.Cu) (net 5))
 (segment (start 122.6257 52) (end 123.8743 52) (width 0.2) (layer F.Cu) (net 5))
 (segment (start 121.3914 52.55) (end 122.6257 52) (width 0.2) (layer F.Cu) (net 5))
 (segment (start 121.35 52.55) (end 121.3914 52.55) (width 0.2) (layer F.Cu) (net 5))
 (segment (start 121.25 52.55) (end 121.35 52.55) (width 0.2) (layer F.Cu) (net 5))
 (segment (start 120.5 52.875) (end 121.25 52.55) (width 0.2) (layer F.Cu) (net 5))
 (segment (start 133.7 51.45) (end 134.45 51.125) (width 0.2) (layer F.Cu) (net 6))
 (segment (start 133.6 51.45) (end 133.7 51.45) (width 0.2) (layer F.Cu) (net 6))
 (segment (start 133.5586 51.45) (end 133.6 51.45) (width 0.2) (layer F.Cu) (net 6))
 (segment (start 132.3743 52) (end 133.5586 51.45) (width 0.2) (layer F.Cu) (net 6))
 (segment (start 131.1257 52) (end 132.3743 52) (width 0.2) (layer F.Cu) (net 6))
 (segment (start 129.8914 52.55) (end 131.1257 52) (width 0.2) (layer F.Cu) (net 6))
 (segment (start 129.85 52.55) (end 129.8914 52.55) (width 0.2) (layer F.Cu) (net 6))
 (segment (start 129.75 52.55) (end 129.85 52.55) (width 0.2) (layer F.Cu) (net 6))
 (segment (start 129 52.875) (end 129.75 52.55) (width 0.2) (layer F.Cu) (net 6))
 (segment (start 142.2 51.45) (end 142.95 51.125) (width 0.2) (layer F.Cu) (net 7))
 (segment (start 142.1 51.45) (end 142.2 51.45) (width 0.2) (layer F.Cu) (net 7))
 (segment (start 142.0586 51.45) (end 142.1 51.45) (width 0.2) (layer F.Cu) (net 7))
 (segment (start 140.8743 52) (end 142.0586 51.45) (width 0.2) (layer F.Cu) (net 7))
 (segment (start 139.6257 52) (end 140.8743 52) (width 0.2) (layer F.Cu) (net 7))
 (segment (start 138.3914 52.55) (end 139.6257 52) (width 0.2) (layer F.Cu) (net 7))
 (segment (start 138.35 52.55) (end 138.3914 52.55) (width 0.2) (layer F.Cu) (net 7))
 (segment (start 138.25 52.55) (end 138.35 52.55) (width 0.2) (layer F.Cu) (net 7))
 (segment (start 137.5 52.875) (end 138.25 52.55) (width 0.2) (layer F.Cu) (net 7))
 (segment (start 153.379 50.7297) (end 153.629 50.7297) (width 0.2) (layer F.Cu) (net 8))
 (segment (start 149.6243 52) (end 153.379 50.7297) (width 0.2) (layer F.Cu) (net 8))
 (segment (start 148.3757 52) (end 149.6243 52) (width 0.2) (layer F.Cu) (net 8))
 (segment (start 146.8914 52.55) (end 148.3757 52) (width 0.2) (layer F.Cu) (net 8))
 (segment (start 146.85 52.55) (end 146.8914 52.55) (width 0.2) (layer F.Cu) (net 8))
 (segment (start 146.75 52.55) (end 146.85 52.55) (width 0.2) (layer F.Cu) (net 8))
 (segment (start 146 52.875) (end 146.75 52.55) (width 0.2) (layer F.Cu) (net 8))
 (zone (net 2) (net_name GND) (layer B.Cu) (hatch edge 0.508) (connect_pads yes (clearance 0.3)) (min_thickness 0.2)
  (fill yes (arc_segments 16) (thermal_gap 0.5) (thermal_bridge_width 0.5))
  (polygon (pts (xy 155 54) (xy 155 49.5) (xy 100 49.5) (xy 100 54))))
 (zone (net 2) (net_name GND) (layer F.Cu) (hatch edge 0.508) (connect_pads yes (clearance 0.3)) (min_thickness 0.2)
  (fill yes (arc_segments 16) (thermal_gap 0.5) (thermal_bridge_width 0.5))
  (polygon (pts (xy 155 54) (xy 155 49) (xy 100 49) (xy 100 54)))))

